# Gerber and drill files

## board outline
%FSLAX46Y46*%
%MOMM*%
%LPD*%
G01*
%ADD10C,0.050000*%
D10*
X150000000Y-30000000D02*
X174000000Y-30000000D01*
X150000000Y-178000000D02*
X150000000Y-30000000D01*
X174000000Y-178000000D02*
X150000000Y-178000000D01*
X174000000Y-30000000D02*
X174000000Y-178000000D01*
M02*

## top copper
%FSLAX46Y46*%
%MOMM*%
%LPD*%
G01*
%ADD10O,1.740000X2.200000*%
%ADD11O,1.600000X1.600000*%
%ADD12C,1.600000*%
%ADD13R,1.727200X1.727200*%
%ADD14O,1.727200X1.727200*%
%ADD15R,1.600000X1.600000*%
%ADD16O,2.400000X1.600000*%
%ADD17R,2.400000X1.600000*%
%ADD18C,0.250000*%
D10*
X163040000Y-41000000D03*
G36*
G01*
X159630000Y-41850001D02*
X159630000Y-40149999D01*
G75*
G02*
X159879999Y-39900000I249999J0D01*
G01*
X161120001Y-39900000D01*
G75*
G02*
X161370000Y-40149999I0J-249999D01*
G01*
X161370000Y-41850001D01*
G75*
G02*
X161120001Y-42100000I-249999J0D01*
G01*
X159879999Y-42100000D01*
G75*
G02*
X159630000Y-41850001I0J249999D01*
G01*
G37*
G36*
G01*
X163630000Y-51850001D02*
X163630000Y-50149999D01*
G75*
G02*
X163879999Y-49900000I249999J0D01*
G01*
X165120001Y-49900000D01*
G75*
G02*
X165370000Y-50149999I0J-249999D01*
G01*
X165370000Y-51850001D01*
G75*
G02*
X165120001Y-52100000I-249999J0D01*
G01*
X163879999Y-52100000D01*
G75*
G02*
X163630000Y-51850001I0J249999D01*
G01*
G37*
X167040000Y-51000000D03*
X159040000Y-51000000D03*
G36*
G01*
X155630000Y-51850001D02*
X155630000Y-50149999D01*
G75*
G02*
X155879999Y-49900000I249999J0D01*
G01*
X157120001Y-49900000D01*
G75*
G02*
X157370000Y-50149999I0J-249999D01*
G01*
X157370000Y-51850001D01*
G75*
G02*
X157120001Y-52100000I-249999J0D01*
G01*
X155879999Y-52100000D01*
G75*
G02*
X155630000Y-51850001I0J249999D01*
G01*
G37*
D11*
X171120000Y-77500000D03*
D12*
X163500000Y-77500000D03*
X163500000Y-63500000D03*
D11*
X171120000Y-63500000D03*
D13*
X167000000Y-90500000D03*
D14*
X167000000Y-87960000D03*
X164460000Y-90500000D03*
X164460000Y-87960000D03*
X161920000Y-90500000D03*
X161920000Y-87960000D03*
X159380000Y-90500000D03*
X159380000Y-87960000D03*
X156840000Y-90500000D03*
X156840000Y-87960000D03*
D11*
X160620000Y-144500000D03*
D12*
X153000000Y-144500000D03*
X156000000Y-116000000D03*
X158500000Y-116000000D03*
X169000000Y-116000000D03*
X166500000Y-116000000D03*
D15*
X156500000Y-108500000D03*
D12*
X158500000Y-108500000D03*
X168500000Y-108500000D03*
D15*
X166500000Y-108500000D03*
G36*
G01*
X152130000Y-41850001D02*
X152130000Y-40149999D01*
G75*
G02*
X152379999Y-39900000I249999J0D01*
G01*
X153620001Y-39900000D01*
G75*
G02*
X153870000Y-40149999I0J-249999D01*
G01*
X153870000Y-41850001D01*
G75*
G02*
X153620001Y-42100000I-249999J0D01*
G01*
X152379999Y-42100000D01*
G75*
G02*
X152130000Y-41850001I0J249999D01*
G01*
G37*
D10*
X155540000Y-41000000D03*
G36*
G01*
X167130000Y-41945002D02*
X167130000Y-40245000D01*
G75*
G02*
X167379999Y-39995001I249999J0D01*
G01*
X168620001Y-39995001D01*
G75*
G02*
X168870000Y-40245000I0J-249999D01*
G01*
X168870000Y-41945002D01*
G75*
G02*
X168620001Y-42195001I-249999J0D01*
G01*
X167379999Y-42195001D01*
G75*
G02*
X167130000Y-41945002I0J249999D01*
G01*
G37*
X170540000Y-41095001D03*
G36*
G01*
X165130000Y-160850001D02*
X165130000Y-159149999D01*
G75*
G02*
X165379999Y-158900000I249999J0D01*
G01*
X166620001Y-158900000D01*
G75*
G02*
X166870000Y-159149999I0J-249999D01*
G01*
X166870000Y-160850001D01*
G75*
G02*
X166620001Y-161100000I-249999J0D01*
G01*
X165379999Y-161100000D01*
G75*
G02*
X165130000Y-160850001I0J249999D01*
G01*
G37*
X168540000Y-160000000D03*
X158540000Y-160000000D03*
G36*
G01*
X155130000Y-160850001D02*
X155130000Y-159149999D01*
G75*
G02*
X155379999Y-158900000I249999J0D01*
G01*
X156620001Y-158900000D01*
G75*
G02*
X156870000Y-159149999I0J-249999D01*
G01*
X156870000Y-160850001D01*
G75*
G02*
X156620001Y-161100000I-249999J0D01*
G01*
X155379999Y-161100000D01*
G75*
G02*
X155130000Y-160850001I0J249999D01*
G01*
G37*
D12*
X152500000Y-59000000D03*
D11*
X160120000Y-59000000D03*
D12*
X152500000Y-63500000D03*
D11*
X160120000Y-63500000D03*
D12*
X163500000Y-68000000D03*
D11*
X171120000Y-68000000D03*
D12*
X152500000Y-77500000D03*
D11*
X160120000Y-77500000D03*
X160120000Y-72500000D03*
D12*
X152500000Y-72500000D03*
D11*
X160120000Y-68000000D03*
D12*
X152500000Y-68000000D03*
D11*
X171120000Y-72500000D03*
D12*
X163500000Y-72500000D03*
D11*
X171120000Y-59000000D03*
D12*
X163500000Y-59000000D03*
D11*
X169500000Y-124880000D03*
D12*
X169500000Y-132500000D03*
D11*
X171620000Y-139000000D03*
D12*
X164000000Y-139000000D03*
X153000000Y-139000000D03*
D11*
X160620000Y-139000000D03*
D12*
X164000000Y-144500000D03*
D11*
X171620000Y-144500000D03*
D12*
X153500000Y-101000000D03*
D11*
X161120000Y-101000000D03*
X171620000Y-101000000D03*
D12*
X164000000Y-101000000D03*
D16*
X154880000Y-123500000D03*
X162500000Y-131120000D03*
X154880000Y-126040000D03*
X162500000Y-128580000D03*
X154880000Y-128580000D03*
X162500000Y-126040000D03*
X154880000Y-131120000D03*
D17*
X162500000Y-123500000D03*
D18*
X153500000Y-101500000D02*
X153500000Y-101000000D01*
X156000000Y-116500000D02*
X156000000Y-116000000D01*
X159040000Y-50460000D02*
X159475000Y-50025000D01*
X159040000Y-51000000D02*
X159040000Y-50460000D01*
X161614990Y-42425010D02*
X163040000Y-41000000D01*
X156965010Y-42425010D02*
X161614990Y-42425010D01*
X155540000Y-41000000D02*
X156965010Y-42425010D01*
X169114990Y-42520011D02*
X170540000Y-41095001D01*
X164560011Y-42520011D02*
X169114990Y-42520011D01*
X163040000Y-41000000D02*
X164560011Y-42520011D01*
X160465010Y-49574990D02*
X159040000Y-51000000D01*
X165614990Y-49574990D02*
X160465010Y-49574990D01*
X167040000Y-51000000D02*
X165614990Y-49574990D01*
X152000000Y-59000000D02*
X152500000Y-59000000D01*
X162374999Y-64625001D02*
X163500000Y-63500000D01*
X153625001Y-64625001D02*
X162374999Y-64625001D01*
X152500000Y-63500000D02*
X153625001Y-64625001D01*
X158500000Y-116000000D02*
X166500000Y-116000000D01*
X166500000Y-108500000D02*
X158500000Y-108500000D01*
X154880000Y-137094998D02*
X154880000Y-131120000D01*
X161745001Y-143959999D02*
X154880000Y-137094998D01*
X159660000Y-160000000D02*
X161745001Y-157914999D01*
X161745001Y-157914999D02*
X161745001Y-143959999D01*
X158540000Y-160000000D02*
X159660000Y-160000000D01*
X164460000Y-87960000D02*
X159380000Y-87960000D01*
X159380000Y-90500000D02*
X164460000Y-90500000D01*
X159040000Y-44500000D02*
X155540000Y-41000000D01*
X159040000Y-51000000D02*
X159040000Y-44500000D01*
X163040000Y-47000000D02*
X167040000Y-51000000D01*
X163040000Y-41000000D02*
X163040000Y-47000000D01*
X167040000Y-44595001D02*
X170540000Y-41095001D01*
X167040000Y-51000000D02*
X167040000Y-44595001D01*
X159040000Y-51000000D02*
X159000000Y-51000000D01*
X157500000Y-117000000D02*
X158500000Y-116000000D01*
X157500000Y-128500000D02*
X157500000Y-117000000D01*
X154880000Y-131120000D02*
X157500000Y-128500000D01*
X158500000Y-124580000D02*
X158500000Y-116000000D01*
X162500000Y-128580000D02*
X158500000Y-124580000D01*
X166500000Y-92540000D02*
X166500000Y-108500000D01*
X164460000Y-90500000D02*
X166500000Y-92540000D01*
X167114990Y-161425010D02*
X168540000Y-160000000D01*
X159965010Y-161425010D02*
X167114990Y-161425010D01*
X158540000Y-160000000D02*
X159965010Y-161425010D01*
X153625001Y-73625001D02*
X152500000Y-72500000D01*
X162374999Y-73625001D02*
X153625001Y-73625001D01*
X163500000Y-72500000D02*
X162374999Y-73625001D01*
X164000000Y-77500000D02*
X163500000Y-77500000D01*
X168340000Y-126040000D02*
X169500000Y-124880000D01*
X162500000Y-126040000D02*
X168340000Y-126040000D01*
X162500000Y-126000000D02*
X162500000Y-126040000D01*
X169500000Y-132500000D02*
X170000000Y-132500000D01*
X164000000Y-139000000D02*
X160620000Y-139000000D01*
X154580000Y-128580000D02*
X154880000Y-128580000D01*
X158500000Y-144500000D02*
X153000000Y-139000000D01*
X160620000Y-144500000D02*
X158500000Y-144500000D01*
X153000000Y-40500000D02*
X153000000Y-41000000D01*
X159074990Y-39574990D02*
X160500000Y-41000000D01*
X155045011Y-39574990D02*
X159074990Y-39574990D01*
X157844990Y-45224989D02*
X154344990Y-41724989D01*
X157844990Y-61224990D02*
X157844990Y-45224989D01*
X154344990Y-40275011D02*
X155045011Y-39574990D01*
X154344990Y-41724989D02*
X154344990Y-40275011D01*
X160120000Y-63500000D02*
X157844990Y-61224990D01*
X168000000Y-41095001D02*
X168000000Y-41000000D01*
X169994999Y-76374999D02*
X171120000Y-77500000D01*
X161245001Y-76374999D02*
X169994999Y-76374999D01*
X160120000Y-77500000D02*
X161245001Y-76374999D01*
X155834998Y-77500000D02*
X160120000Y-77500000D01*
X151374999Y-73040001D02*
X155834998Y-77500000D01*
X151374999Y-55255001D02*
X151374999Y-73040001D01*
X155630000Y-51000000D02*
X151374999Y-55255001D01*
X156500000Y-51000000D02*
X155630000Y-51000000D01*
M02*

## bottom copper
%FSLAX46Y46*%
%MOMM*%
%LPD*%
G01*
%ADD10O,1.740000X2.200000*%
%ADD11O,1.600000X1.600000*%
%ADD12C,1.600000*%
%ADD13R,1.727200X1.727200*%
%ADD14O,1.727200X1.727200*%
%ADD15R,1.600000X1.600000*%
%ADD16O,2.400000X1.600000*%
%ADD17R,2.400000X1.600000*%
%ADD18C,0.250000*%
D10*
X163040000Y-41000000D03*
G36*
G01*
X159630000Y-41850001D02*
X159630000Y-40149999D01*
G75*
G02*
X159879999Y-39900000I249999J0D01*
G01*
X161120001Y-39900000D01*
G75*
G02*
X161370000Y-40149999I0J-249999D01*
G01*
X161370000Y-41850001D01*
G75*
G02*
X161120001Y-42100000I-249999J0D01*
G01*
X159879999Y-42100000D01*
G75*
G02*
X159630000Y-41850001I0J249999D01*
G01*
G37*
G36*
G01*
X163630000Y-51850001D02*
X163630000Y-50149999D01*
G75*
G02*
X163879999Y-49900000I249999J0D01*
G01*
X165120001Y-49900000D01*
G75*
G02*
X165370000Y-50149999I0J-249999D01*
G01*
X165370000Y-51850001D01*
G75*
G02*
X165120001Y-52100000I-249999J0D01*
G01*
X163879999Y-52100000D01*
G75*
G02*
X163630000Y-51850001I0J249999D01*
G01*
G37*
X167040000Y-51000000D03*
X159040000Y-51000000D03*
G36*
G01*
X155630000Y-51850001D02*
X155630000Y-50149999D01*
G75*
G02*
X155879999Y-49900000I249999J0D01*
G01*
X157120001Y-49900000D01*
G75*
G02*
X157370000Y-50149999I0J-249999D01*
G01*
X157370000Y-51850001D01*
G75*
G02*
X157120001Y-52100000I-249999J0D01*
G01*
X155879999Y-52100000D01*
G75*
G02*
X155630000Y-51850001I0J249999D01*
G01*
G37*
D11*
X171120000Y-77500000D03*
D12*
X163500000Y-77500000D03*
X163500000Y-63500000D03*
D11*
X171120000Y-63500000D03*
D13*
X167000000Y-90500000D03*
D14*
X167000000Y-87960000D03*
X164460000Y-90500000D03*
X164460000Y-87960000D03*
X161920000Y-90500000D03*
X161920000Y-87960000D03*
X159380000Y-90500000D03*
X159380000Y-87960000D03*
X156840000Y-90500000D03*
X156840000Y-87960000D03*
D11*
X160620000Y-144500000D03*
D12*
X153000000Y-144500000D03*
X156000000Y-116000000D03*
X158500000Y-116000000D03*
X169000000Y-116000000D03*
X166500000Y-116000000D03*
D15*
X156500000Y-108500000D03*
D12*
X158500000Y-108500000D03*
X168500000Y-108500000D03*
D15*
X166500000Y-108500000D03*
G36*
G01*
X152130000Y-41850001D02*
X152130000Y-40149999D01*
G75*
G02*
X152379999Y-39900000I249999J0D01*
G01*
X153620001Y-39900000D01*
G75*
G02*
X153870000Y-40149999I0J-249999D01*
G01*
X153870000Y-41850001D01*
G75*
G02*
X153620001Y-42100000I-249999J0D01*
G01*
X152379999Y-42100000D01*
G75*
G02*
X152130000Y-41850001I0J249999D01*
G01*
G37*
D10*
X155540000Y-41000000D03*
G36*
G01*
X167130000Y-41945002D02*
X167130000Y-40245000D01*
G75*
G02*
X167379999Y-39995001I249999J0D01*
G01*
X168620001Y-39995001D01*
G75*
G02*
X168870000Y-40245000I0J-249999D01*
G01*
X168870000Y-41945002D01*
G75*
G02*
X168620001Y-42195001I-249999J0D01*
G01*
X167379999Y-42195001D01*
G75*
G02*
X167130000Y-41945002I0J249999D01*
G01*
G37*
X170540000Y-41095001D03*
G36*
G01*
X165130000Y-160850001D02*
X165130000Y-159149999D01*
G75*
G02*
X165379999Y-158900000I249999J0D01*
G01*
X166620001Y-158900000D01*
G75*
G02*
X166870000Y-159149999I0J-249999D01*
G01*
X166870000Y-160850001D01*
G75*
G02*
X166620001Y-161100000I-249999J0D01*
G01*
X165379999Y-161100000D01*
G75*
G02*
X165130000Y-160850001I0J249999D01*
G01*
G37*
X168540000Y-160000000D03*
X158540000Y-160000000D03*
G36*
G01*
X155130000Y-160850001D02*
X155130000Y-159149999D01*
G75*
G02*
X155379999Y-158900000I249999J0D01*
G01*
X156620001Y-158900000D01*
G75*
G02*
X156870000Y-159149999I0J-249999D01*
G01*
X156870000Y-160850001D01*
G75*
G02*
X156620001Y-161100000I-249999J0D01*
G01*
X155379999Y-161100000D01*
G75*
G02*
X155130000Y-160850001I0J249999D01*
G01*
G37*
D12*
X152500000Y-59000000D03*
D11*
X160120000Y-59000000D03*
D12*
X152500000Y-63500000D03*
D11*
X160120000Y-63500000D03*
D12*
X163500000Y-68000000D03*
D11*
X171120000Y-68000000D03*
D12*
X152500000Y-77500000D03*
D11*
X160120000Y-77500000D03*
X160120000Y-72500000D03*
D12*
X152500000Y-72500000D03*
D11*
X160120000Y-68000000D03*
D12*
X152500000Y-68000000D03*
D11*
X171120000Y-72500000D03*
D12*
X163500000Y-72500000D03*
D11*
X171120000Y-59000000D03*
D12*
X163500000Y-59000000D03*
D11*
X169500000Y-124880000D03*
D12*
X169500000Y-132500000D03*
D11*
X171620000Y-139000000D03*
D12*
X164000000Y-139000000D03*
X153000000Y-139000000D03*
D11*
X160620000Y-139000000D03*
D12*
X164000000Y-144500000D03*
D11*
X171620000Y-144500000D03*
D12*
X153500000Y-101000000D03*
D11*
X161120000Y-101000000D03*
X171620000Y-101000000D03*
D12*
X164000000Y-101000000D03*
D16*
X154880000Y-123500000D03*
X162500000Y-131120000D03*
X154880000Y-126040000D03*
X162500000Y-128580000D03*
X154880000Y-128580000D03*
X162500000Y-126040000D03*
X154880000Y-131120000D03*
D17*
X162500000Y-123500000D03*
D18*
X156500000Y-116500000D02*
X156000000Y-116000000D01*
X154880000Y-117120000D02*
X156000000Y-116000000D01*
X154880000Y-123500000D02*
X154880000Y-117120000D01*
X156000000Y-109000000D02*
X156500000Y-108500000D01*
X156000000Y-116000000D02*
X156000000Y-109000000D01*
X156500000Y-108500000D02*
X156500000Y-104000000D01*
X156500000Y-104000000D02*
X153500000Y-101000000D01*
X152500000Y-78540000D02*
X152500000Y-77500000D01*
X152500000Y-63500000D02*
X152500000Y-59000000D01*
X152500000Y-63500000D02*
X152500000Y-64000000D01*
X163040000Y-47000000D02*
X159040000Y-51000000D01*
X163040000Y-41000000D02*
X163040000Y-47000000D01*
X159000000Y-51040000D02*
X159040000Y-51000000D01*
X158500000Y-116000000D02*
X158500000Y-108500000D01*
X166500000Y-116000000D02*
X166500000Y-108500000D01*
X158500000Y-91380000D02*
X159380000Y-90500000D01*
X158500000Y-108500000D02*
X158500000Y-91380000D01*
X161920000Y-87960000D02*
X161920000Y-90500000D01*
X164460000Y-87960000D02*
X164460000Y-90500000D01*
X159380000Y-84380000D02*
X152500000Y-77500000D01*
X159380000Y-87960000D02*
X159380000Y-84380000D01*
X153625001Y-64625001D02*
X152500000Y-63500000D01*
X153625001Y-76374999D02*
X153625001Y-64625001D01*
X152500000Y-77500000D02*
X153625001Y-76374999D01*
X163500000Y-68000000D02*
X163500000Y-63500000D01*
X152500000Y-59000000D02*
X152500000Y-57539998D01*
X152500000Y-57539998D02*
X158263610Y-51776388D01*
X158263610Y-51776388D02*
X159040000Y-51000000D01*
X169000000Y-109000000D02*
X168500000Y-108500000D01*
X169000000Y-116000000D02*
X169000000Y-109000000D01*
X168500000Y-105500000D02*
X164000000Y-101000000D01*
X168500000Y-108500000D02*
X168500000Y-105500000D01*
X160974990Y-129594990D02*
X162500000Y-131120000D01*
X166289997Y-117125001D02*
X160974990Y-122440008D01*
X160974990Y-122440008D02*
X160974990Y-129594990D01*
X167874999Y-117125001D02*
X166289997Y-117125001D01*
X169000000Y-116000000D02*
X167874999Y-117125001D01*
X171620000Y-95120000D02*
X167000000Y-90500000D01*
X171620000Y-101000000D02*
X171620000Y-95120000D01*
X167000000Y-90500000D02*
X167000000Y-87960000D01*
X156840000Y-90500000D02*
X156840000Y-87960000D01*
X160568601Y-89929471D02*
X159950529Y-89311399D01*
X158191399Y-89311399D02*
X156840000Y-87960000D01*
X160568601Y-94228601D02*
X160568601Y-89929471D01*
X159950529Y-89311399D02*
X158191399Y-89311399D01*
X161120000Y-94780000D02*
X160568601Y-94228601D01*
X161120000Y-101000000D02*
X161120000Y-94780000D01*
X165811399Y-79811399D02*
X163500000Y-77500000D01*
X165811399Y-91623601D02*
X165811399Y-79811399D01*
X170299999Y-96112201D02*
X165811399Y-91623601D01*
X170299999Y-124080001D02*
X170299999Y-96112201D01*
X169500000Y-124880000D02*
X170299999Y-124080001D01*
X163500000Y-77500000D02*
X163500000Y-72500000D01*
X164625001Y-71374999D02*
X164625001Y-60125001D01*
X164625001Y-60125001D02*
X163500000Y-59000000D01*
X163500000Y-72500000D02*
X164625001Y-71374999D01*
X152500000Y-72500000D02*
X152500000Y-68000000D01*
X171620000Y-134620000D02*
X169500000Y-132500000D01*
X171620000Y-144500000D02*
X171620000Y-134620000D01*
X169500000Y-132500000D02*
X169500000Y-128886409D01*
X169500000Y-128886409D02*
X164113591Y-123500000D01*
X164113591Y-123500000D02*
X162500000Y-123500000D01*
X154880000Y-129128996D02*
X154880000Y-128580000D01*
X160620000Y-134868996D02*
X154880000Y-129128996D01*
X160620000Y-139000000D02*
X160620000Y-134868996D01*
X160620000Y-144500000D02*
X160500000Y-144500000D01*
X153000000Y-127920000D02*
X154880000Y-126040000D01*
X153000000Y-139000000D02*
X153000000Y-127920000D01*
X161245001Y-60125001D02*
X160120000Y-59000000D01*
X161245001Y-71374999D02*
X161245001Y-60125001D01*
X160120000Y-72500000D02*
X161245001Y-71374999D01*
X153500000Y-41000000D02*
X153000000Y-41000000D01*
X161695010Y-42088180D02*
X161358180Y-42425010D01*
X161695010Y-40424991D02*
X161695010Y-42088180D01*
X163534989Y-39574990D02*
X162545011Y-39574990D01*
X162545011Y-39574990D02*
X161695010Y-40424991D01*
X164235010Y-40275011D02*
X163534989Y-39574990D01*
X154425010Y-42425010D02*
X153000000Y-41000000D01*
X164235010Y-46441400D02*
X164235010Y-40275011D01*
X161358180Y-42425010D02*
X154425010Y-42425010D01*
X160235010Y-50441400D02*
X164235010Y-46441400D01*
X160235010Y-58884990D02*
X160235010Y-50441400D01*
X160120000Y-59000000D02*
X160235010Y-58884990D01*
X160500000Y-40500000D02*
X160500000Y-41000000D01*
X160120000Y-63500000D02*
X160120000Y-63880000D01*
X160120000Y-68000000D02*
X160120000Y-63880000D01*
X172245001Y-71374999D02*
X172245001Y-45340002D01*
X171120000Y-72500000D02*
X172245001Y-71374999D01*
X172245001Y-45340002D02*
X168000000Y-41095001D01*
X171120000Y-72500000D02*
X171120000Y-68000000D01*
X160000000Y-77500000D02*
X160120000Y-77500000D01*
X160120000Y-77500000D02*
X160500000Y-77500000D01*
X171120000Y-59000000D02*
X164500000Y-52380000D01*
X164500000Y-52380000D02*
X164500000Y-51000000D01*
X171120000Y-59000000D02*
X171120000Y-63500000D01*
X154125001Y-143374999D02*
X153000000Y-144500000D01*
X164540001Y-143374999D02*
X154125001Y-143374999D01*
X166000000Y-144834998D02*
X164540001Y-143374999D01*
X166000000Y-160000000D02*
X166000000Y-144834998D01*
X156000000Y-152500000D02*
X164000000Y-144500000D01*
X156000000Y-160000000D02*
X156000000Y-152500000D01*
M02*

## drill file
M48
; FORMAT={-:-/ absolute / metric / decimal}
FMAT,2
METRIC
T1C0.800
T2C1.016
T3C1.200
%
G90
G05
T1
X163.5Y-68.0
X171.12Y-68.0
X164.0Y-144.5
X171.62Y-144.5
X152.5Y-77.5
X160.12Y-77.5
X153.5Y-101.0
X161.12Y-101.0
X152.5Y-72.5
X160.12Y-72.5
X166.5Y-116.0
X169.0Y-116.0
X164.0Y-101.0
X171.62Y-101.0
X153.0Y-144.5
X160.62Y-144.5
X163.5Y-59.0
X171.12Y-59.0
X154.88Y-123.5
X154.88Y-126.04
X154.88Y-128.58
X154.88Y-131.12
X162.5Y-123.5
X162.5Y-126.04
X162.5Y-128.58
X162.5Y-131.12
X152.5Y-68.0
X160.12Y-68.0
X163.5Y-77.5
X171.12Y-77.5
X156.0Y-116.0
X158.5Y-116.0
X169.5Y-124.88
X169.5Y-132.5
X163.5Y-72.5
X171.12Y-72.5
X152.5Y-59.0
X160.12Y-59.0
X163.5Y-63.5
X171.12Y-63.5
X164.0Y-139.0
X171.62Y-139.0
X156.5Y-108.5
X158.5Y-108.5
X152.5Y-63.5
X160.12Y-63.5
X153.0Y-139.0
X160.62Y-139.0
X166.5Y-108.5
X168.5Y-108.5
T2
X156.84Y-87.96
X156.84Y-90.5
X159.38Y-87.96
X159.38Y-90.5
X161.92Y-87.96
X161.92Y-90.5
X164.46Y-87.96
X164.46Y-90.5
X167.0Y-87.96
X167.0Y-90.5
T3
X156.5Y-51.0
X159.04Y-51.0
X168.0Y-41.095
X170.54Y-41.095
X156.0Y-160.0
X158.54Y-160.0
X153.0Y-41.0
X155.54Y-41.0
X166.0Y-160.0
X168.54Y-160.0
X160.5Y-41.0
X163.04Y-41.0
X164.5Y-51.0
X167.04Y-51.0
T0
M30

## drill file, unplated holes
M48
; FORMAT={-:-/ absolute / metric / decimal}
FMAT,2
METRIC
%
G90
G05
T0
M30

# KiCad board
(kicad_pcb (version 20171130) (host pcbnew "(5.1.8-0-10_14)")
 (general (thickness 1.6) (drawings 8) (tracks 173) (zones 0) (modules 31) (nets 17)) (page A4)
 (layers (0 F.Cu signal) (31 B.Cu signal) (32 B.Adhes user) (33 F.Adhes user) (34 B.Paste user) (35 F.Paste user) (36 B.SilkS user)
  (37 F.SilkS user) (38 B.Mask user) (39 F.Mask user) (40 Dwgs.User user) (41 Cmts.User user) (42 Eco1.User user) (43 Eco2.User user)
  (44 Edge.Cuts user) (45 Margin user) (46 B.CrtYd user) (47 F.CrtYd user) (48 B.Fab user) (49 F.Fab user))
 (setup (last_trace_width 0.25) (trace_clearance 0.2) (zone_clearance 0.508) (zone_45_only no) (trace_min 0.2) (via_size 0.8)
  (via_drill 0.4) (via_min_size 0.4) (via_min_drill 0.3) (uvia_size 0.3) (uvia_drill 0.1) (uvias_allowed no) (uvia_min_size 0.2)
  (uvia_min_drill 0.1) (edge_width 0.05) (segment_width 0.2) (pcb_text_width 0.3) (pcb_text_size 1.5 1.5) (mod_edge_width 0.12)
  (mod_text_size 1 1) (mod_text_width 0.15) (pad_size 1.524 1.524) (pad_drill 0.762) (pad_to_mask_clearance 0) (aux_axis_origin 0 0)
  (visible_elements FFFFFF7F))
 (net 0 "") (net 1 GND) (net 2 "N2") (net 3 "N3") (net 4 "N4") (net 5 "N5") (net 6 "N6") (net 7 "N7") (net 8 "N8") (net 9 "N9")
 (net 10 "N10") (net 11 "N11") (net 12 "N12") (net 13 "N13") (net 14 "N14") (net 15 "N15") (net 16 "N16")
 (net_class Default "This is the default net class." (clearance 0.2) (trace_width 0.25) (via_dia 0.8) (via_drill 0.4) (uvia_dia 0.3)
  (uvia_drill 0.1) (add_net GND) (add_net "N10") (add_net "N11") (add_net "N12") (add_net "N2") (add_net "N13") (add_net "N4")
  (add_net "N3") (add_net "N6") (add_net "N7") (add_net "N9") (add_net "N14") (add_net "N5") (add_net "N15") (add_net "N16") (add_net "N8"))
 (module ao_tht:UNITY (layer F.Cu) (at 162 105 270)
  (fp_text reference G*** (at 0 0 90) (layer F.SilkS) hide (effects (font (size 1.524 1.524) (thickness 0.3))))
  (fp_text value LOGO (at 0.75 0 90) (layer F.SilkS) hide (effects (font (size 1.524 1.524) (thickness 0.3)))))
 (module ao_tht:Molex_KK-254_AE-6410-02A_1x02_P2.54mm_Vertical (layer F.Cu) (at 160.5 41)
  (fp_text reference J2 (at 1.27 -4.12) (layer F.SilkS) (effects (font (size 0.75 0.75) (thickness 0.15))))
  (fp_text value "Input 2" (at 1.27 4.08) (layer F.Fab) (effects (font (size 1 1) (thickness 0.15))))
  (pad 2 thru_hole oval (at 2.54 0) (size 1.74 2.2) (drill 1.2) (layers *.Cu *.Mask) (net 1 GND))
  (pad 1 thru_hole roundrect (at 0 0) (size 1.74 2.2) (drill 1.2) (layers *.Cu *.Mask) (roundrect_rratio 0.1436775862068966) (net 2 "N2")))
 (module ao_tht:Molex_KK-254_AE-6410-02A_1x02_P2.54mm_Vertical (layer F.Cu) (at 164.5 51)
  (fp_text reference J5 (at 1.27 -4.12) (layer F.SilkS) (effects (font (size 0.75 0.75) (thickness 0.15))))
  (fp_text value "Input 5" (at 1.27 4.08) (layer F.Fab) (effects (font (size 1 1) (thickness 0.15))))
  (pad 1 thru_hole roundrect (at 0 0) (size 1.74 2.2) (drill 1.2) (layers *.Cu *.Mask) (roundrect_rratio 0.1436775862068966) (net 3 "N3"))
  (pad 2 thru_hole oval (at 2.54 0) (size 1.74 2.2) (drill 1.2) (layers *.Cu *.Mask) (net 1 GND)))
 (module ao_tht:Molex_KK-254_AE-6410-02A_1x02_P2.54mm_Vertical (layer F.Cu) (at 156.5 51)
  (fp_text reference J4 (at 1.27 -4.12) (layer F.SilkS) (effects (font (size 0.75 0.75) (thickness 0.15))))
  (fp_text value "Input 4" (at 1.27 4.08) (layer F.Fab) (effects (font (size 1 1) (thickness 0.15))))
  (pad 2 thru_hole oval (at 2.54 0) (size 1.74 2.2) (drill 1.2) (layers *.Cu *.Mask) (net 1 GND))
  (pad 1 thru_hole roundrect (at 0 0) (size 1.74 2.2) (drill 1.2) (layers *.Cu *.Mask) (roundrect_rratio 0.1436775862068966) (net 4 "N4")))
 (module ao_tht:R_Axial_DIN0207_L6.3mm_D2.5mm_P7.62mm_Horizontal (layer B.Cu) (at 163.5 77.5)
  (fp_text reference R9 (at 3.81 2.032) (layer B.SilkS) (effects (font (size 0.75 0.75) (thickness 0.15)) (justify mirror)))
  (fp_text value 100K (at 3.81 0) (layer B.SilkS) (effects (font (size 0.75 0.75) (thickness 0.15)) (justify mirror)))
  (pad 2 thru_hole oval (at 7.62 0) (size 1.6 1.6) (drill 0.8) (layers *.Cu *.Mask) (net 4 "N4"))
  (pad 1 thru_hole circle (at 0 0) (size 1.6 1.6) (drill 0.8) (layers *.Cu *.Mask) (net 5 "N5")))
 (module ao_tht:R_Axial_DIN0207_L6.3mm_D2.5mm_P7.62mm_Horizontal (layer B.Cu) (at 163.5 63.5)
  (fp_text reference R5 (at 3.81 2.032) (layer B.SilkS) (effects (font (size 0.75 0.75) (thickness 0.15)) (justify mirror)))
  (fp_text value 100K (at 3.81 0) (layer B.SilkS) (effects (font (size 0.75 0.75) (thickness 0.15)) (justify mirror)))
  (pad 1 thru_hole circle (at 0 0) (size 1.6 1.6) (drill 0.8) (layers *.Cu *.Mask) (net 1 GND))
  (pad 2 thru_hole oval (at 7.62 0) (size 1.6 1.6) (drill 0.8) (layers *.Cu *.Mask) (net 3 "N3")))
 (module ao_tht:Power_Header (layer B.Cu) (at 167 90.5 90)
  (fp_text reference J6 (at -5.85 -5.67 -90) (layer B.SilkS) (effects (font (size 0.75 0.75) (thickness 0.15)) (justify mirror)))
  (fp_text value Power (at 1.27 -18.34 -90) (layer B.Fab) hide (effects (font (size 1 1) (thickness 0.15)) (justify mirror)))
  (pad 1 thru_hole rect (at 0 0 90) (size 1.7272 1.7272) (drill 1.016) (layers *.Cu *.Mask) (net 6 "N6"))
  (pad 2 thru_hole oval (at 2.54 0 90) (size 1.7272 1.7272) (drill 1.016) (layers *.Cu *.Mask) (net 6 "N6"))
  (pad 3 thru_hole oval (at 0 -2.54 90) (size 1.7272 1.7272) (drill 1.016) (layers *.Cu *.Mask) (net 1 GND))
  (pad 4 thru_hole oval (at 2.54 -2.54 90) (size 1.7272 1.7272) (drill 1.016) (layers *.Cu *.Mask) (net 1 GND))
  (pad 5 thru_hole oval (at 0 -5.08 90) (size 1.7272 1.7272) (drill 1.016) (layers *.Cu *.Mask) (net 1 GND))
  (pad 6 thru_hole oval (at 2.54 -5.08 90) (size 1.7272 1.7272) (drill 1.016) (layers *.Cu *.Mask) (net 1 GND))
  (pad 7 thru_hole oval (at 0 -7.62 90) (size 1.7272 1.7272) (drill 1.016) (layers *.Cu *.Mask) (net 1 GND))
  (pad 8 thru_hole oval (at 2.54 -7.62 90) (size 1.7272 1.7272) (drill 1.016) (layers *.Cu *.Mask) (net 1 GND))
  (pad 9 thru_hole oval (at 0 -10.16 90) (size 1.7272 1.7272) (drill 1.016) (layers *.Cu *.Mask) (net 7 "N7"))
  (pad 10 thru_hole oval (at 2.54 -10.16 90) (size 1.7272 1.7272) (drill 1.016) (layers *.Cu *.Mask) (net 7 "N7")))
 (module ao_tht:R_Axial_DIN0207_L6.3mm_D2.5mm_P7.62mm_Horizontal (layer B.Cu) (at 153 144.5)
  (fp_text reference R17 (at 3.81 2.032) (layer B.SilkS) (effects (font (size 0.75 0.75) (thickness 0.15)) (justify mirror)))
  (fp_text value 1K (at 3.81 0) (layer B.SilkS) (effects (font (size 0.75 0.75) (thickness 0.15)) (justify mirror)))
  (pad 2 thru_hole oval (at 7.62 0) (size 1.6 1.6) (drill 0.8) (layers *.Cu *.Mask) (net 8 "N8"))
  (pad 1 thru_hole circle (at 0 0) (size 1.6 1.6) (drill 0.8) (layers *.Cu *.Mask) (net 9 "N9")))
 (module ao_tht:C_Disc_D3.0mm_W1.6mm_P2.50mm (layer B.Cu) (at 156 116)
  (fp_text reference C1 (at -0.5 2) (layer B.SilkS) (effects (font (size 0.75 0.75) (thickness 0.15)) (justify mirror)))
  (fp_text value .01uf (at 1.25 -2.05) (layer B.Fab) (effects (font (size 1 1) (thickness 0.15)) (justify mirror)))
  (pad 1 thru_hole circle (at 0 0) (size 1.6 1.6) (drill 0.8) (layers *.Cu *.Mask) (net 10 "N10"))
  (pad 2 thru_hole circle (at 2.5 0) (size 1.6 1.6) (drill 0.8) (layers *.Cu *.Mask) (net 1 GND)))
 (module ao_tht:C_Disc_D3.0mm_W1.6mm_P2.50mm (layer B.Cu) (at 166.5 116)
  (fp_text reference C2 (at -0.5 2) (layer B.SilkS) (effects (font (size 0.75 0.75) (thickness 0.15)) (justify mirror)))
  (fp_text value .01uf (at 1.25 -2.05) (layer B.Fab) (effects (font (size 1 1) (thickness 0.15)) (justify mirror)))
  (pad 2 thru_hole circle (at 2.5 0) (size 1.6 1.6) (drill 0.8) (layers *.Cu *.Mask) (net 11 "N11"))
  (pad 1 thru_hole circle (at 0 0) (size 1.6 1.6) (drill 0.8) (layers *.Cu *.Mask) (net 1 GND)))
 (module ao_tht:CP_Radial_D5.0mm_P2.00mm (layer B.Cu) (at 156.5 108.5)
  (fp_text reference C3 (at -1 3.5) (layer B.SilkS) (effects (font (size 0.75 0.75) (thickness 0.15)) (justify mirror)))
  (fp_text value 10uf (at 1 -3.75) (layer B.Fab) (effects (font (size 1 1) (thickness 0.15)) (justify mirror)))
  (pad 1 thru_hole rect (at 0 0) (size 1.6 1.6) (drill 0.8) (layers *.Cu *.Mask) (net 10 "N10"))
  (pad 2 thru_hole circle (at 2 0) (size 1.6 1.6) (drill 0.8) (layers *.Cu *.Mask) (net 1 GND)))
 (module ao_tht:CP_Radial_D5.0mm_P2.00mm (layer B.Cu) (at 166.5 108.5)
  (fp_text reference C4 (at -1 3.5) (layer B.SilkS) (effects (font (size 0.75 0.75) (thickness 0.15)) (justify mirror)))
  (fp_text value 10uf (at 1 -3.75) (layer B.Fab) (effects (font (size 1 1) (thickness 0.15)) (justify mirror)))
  (pad 2 thru_hole circle (at 2 0) (size 1.6 1.6) (drill 0.8) (layers *.Cu *.Mask) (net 11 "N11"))
  (pad 1 thru_hole rect (at 0 0) (size 1.6 1.6) (drill 0.8) (layers *.Cu *.Mask) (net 1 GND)))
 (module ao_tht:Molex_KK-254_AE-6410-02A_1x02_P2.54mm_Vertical (layer F.Cu) (at 153 41)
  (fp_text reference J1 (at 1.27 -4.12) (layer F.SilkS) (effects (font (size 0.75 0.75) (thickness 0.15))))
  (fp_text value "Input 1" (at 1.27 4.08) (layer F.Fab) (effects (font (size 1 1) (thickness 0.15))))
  (pad 1 thru_hole roundrect (at 0 0) (size 1.74 2.2) (drill 1.2) (layers *.Cu *.Mask) (roundrect_rratio 0.1436775862068966) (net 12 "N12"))
  (pad 2 thru_hole oval (at 2.54 0) (size 1.74 2.2) (drill 1.2) (layers *.Cu *.Mask) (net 1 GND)))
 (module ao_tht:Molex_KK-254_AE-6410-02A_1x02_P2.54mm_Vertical (layer F.Cu) (at 168 41.095001)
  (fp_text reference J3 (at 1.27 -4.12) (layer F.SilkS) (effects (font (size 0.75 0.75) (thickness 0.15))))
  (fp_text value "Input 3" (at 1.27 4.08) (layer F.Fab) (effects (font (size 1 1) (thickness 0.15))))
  (pad 1 thru_hole roundrect (at 0 0) (size 1.74 2.2) (drill 1.2) (layers *.Cu *.Mask) (roundrect_rratio 0.1436775862068966) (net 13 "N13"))
  (pad 2 thru_hole oval (at 2.54 0) (size 1.74 2.2) (drill 1.2) (layers *.Cu *.Mask) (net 1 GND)))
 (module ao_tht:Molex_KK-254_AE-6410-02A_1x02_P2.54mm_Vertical (layer F.Cu) (at 166 160)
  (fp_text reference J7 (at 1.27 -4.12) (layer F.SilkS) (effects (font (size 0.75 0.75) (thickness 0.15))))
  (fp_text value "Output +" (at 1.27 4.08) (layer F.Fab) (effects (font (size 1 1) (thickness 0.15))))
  (pad 1 thru_hole roundrect (at 0 0) (size 1.74 2.2) (drill 1.2) (layers *.Cu *.Mask) (roundrect_rratio 0.1436775862068966) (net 9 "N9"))
  (pad 2 thru_hole oval (at 2.54 0) (size 1.74 2.2) (drill 1.2) (layers *.Cu *.Mask) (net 1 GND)))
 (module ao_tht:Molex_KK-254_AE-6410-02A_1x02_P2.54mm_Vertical (layer F.Cu) (at 156 160)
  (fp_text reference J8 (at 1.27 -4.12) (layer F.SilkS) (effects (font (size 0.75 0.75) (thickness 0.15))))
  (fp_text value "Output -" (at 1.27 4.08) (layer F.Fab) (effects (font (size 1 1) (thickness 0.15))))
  (pad 2 thru_hole oval (at 2.54 0) (size 1.74 2.2) (drill 1.2) (layers *.Cu *.Mask) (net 1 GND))
  (pad 1 thru_hole roundrect (at 0 0) (size 1.74 2.2) (drill 1.2) (layers *.Cu *.Mask) (roundrect_rratio 0.1436775862068966) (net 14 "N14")))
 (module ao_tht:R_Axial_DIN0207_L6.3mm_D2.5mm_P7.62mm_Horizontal (layer B.Cu) (at 152.5 59)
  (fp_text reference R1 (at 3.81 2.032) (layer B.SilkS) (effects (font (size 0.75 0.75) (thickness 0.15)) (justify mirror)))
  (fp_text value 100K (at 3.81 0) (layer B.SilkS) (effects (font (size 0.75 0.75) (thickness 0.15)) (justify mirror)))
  (pad 1 thru_hole circle (at 0 0) (size 1.6 1.6) (drill 0.8) (layers *.Cu *.Mask) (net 1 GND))
  (pad 2 thru_hole oval (at 7.62 0) (size 1.6 1.6) (drill 0.8) (layers *.Cu *.Mask) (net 12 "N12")))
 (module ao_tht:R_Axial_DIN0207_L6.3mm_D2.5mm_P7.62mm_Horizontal (layer B.Cu) (at 152.5 63.5)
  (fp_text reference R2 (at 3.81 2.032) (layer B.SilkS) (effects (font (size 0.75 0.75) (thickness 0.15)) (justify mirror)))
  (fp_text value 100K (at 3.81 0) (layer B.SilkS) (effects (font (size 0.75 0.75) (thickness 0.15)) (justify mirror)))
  (pad 1 thru_hole circle (at 0 0) (size 1.6 1.6) (drill 0.8) (layers *.Cu *.Mask) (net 1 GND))
  (pad 2 thru_hole oval (at 7.62 0) (size 1.6 1.6) (drill 0.8) (layers *.Cu *.Mask) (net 2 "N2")))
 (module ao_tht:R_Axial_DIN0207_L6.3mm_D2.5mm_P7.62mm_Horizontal (layer B.Cu) (at 163.5 68)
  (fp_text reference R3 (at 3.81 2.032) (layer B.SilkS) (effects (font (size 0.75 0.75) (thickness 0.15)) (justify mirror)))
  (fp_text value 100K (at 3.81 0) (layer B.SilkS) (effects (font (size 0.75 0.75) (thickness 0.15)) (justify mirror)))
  (pad 1 thru_hole circle (at 0 0) (size 1.6 1.6) (drill 0.8) (layers *.Cu *.Mask) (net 1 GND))
  (pad 2 thru_hole oval (at 7.62 0) (size 1.6 1.6) (drill 0.8) (layers *.Cu *.Mask) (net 13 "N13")))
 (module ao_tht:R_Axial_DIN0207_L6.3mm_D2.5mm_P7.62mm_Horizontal (layer B.Cu) (at 152.5 77.5)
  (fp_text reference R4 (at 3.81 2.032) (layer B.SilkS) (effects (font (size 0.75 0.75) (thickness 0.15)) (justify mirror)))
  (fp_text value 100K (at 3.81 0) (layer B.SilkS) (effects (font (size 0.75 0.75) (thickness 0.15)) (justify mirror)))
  (pad 1 thru_hole circle (at 0 0) (size 1.6 1.6) (drill 0.8) (layers *.Cu *.Mask) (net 1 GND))
  (pad 2 thru_hole oval (at 7.62 0) (size 1.6 1.6) (drill 0.8) (layers *.Cu *.Mask) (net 4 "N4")))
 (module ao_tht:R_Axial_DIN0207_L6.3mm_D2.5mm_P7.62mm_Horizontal (layer B.Cu) (at 152.5 72.5)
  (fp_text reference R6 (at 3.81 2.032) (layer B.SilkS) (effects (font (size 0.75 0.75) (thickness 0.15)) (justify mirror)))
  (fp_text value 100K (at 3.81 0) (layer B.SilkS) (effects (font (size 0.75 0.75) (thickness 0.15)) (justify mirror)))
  (pad 2 thru_hole oval (at 7.62 0) (size 1.6 1.6) (drill 0.8) (layers *.Cu *.Mask) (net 12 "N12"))
  (pad 1 thru_hole circle (at 0 0) (size 1.6 1.6) (drill 0.8) (layers *.Cu *.Mask) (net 5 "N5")))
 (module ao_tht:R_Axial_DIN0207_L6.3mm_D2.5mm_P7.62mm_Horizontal (layer B.Cu) (at 152.5 68)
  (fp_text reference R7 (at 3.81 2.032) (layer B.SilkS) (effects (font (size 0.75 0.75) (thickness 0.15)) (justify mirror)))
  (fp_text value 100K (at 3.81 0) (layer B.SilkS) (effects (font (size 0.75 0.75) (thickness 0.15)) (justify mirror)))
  (pad 2 thru_hole oval (at 7.62 0) (size 1.6 1.6) (drill 0.8) (layers *.Cu *.Mask) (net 2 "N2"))
  (pad 1 thru_hole circle (at 0 0) (size 1.6 1.6) (drill 0.8) (layers *.Cu *.Mask) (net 5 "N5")))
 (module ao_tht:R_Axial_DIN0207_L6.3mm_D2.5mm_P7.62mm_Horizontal (layer B.Cu) (at 163.5 72.5)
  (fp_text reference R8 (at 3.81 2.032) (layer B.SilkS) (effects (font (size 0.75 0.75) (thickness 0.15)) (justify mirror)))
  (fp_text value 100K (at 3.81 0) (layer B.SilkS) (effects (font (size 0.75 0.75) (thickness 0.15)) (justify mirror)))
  (pad 2 thru_hole oval (at 7.62 0) (size 1.6 1.6) (drill 0.8) (layers *.Cu *.Mask) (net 13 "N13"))
  (pad 1 thru_hole circle (at 0 0) (size 1.6 1.6) (drill 0.8) (layers *.Cu *.Mask) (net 5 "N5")))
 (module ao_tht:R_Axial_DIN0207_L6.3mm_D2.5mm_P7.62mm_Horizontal (layer B.Cu) (at 163.5 59)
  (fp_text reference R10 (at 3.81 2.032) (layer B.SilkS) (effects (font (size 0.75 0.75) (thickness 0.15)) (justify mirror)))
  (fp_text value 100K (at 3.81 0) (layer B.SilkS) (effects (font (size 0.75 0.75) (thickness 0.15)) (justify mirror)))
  (pad 2 thru_hole oval (at 7.62 0) (size 1.6 1.6) (drill 0.8) (layers *.Cu *.Mask) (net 3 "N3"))
  (pad 1 thru_hole circle (at 0 0) (size 1.6 1.6) (drill 0.8) (layers *.Cu *.Mask) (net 5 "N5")))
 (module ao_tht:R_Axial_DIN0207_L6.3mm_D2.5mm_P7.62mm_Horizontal (layer B.Cu) (at 169.5 132.5 90)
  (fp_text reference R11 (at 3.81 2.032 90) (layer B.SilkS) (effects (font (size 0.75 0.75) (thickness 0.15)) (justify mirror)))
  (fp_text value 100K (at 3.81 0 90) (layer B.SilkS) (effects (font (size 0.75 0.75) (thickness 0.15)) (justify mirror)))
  (pad 2 thru_hole oval (at 7.62 0 90) (size 1.6 1.6) (drill 0.8) (layers *.Cu *.Mask) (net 5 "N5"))
  (pad 1 thru_hole circle (at 0 0 90) (size 1.6 1.6) (drill 0.8) (layers *.Cu *.Mask) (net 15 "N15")))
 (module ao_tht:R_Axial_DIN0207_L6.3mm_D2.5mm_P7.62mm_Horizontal (layer B.Cu) (at 164 139)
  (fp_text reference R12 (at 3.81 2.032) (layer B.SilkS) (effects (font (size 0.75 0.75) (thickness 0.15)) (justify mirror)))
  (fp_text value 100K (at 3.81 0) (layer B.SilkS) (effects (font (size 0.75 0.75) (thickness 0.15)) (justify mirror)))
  (pad 2 thru_hole oval (at 7.62 0) (size 1.6 1.6) (drill 0.8) (layers *.Cu *.Mask) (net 15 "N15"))
  (pad 1 thru_hole circle (at 0 0) (size 1.6 1.6) (drill 0.8) (layers *.Cu *.Mask) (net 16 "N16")))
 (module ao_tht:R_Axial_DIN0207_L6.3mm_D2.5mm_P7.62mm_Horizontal (layer B.Cu) (at 153 139)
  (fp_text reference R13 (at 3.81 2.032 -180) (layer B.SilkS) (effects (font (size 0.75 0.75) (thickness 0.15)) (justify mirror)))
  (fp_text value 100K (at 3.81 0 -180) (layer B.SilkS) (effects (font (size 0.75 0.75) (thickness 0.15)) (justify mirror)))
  (pad 1 thru_hole circle (at 0 0) (size 1.6 1.6) (drill 0.8) (layers *.Cu *.Mask) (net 8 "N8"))
  (pad 2 thru_hole oval (at 7.62 0) (size 1.6 1.6) (drill 0.8) (layers *.Cu *.Mask) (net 16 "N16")))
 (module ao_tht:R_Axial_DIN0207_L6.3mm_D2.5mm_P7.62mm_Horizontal (layer B.Cu) (at 164 144.5)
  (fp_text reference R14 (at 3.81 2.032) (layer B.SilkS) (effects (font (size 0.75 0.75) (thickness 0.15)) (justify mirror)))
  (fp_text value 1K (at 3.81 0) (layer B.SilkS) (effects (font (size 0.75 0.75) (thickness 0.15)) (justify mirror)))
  (pad 1 thru_hole circle (at 0 0) (size 1.6 1.6) (drill 0.8) (layers *.Cu *.Mask) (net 14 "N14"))
  (pad 2 thru_hole oval (at 7.62 0) (size 1.6 1.6) (drill 0.8) (layers *.Cu *.Mask) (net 15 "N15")))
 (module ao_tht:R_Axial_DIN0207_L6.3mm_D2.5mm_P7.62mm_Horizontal (layer B.Cu) (at 153.5 101)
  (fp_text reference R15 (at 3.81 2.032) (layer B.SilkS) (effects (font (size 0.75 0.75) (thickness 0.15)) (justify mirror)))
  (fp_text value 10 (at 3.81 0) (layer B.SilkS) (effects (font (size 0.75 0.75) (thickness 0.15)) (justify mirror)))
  (pad 1 thru_hole circle (at 0 0) (size 1.6 1.6) (drill 0.8) (layers *.Cu *.Mask) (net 10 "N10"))
  (pad 2 thru_hole oval (at 7.62 0) (size 1.6 1.6) (drill 0.8) (layers *.Cu *.Mask) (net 7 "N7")))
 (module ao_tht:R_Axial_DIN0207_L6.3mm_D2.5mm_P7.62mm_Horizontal (layer B.Cu) (at 164 101)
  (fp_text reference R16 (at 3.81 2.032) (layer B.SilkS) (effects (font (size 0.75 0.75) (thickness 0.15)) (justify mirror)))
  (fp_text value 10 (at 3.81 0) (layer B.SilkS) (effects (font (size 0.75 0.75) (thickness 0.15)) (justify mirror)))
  (pad 2 thru_hole oval (at 7.62 0) (size 1.6 1.6) (drill 0.8) (layers *.Cu *.Mask) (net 6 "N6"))
  (pad 1 thru_hole circle (at 0 0) (size 1.6 1.6) (drill 0.8) (layers *.Cu *.Mask) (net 11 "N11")))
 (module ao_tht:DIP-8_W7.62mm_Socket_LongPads (layer B.Cu) (at 162.5 123.5 180)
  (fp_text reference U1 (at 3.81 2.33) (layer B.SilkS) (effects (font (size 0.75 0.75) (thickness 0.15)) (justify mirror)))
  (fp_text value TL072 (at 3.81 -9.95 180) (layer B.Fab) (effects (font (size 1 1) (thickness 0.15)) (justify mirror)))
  (pad 8 thru_hole oval (at 7.62 0 180) (size 2.4 1.6) (drill 0.8) (layers *.Cu *.Mask) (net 10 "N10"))
  (pad 4 thru_hole oval (at 0 -7.62 180) (size 2.4 1.6) (drill 0.8) (layers *.Cu *.Mask) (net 11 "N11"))
  (pad 7 thru_hole oval (at 7.62 -2.54 180) (size 2.4 1.6) (drill 0.8) (layers *.Cu *.Mask) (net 8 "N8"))
  (pad 3 thru_hole oval (at 0 -5.08 180) (size 2.4 1.6) (drill 0.8) (layers *.Cu *.Mask) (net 1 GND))
  (pad 6 thru_hole oval (at 7.62 -5.08 180) (size 2.4 1.6) (drill 0.8) (layers *.Cu *.Mask) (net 16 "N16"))
  (pad 2 thru_hole oval (at 0 -2.54 180) (size 2.4 1.6) (drill 0.8) (layers *.Cu *.Mask) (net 5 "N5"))
  (pad 5 thru_hole oval (at 7.62 -7.62 180) (size 2.4 1.6) (drill 0.8) (layers *.Cu *.Mask) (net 1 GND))
  (pad 1 thru_hole rect (at 0 0 180) (size 2.4 1.6) (drill 0.8) (layers *.Cu *.Mask) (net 15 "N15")))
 (gr_line (start 150 30) (end 174 30) (layer Edge.Cuts) (width 0.05))
 (gr_line (start 150 178) (end 150 30) (layer Edge.Cuts) (width 0.05))
 (gr_line (start 174 178) (end 150 178) (layer Edge.Cuts) (width 0.05))
 (gr_line (start 174 30) (end 174 178) (layer Edge.Cuts) (width 0.05))
 (segment (start 156.5 116.5) (end 156 116) (width 0.25) (layer B.Cu) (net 10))
 (segment (start 153.5 101.5) (end 153.5 101) (width 0.25) (layer F.Cu) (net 10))
 (segment (start 156 116.5) (end 156 116) (width 0.25) (layer F.Cu) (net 10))
 (segment (start 154.88 117.12) (end 156 116) (width 0.25) (layer B.Cu) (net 10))
 (segment (start 154.88 123.5) (end 154.88 117.12) (width 0.25) (layer B.Cu) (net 10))
 (segment (start 156 109) (end 156.5 108.5) (width 0.25) (layer B.Cu) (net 10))
 (segment (start 156 116) (end 156 109) (width 0.25) (layer B.Cu) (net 10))
 (segment (start 156.5 108.5) (end 156.5 104) (width 0.25) (layer B.Cu) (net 10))
 (segment (start 156.5 104) (end 153.5 101) (width 0.25) (layer B.Cu) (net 10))
 (segment (start 159.04 50.46) (end 159.475 50.025) (width 0.25) (layer F.Cu) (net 1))
 (segment (start 159.04 51) (end 159.04 50.46) (width 0.25) (layer F.Cu) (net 1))
 (segment (start 152.5 78.54) (end 152.5 77.5) (width 0.25) (layer B.Cu) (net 1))
 (segment (start 152.5 63.5) (end 152.5 59) (width 0.25) (layer B.Cu) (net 1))
 (segment (start 152.5 63.5) (end 152.5 64) (width 0.25) (layer B.Cu) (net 1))
 (segment (start 163.04 47) (end 159.04 51) (width 0.25) (layer B.Cu) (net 1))
 (segment (start 163.04 41) (end 163.04 47) (width 0.25) (layer B.Cu) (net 1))
 (segment (start 159 51.04) (end 159.04 51) (width 0.25) (layer B.Cu) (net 1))
 (segment (start 161.61499 42.42501) (end 163.04 41) (width 0.25) (layer F.Cu) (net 1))
 (segment (start 156.96501 42.42501) (end 161.61499 42.42501) (width 0.25) (layer F.Cu) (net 1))
 (segment (start 155.54 41) (end 156.96501 42.42501) (width 0.25) (layer F.Cu) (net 1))
 (segment (start 169.11499 42.520011) (end 170.54 41.095001) (width 0.25) (layer F.Cu) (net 1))
 (segment (start 164.560011 42.520011) (end 169.11499 42.520011) (width 0.25) (layer F.Cu) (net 1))
 (segment (start 163.04 41) (end 164.560011 42.520011) (width 0.25) (layer F.Cu) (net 1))
 (segment (start 160.46501 49.57499) (end 159.04 51) (width 0.25) (layer F.Cu) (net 1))
 (segment (start 165.61499 49.57499) (end 160.46501 49.57499) (width 0.25) (layer F.Cu) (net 1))
 (segment (start 167.04 51) (end 165.61499 49.57499) (width 0.25) (layer F.Cu) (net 1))
 (segment (start 152 59) (end 152.5 59) (width 0.25) (layer F.Cu) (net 1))
 (segment (start 162.374999 64.625001) (end 163.5 63.5) (width 0.25) (layer F.Cu) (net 1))
 (segment (start 153.625001 64.625001) (end 162.374999 64.625001) (width 0.25) (layer F.Cu) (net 1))
 (segment (start 152.5 63.5) (end 153.625001 64.625001) (width 0.25) (layer F.Cu) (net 1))
 (segment (start 158.5 116) (end 166.5 116) (width 0.25) (layer F.Cu) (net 1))
 (segment (start 166.5 108.5) (end 158.5 108.5) (width 0.25) (layer F.Cu) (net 1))
 (segment (start 154.88 137.094998) (end 154.88 131.12) (width 0.25) (layer F.Cu) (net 1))
 (segment (start 161.745001 143.959999) (end 154.88 137.094998) (width 0.25) (layer F.Cu) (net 1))
 (segment (start 159.66 160) (end 161.745001 157.914999) (width 0.25) (layer F.Cu) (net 1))
 (segment (start 161.745001 157.914999) (end 161.745001 143.959999) (width 0.25) (layer F.Cu) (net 1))
 (segment (start 158.54 160) (end 159.66 160) (width 0.25) (layer F.Cu) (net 1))
 (segment (start 158.5 116) (end 158.5 108.5) (width 0.25) (layer B.Cu) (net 1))
 (segment (start 166.5 116) (end 166.5 108.5) (width 0.25) (layer B.Cu) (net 1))
 (segment (start 158.5 91.38) (end 159.38 90.5) (width 0.25) (layer B.Cu) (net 1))
 (segment (start 158.5 108.5) (end 158.5 91.38) (width 0.25) (layer B.Cu) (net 1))
 (segment (start 164.46 87.96) (end 159.38 87.96) (width 0.25) (layer F.Cu) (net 1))
 (segment (start 159.38 90.5) (end 164.46 90.5) (width 0.25) (layer F.Cu) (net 1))
 (segment (start 161.92 87.96) (end 161.92 90.5) (width 0.25) (layer B.Cu) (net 1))
 (segment (start 164.46 87.96) (end 164.46 90.5) (width 0.25) (layer B.Cu) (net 1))
 (segment (start 159.38 84.38) (end 152.5 77.5) (width 0.25) (layer B.Cu) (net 1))
 (segment (start 159.38 87.96) (end 159.38 84.38) (width 0.25) (layer B.Cu) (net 1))
 (segment (start 153.625001 64.625001) (end 152.5 63.5) (width 0.25) (layer B.Cu) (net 1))
 (segment (start 153.625001 76.374999) (end 153.625001 64.625001) (width 0.25) (layer B.Cu) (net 1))
 (segment (start 152.5 77.5) (end 153.625001 76.374999) (width 0.25) (layer B.Cu) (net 1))
 (segment (start 163.5 68) (end 163.5 63.5) (width 0.25) (layer B.Cu) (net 1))
 (segment (start 152.5 59) (end 152.5 57.539998) (width 0.25) (layer B.Cu) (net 1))
 (segment (start 152.5 57.539998) (end 158.26361 51.776388) (width 0.25) (layer B.Cu) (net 1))
 (segment (start 158.26361 51.776388) (end 159.04 51) (width 0.25) (layer B.Cu) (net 1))
 (segment (start 159.04 44.5) (end 155.54 41) (width 0.25) (layer F.Cu) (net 1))
 (segment (start 159.04 51) (end 159.04 44.5) (width 0.25) (layer F.Cu) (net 1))
 (segment (start 163.04 47) (end 167.04 51) (width 0.25) (layer F.Cu) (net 1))
 (segment (start 163.04 41) (end 163.04 47) (width 0.25) (layer F.Cu) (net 1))
 (segment (start 167.04 44.595001) (end 170.54 41.095001) (width 0.25) (layer F.Cu) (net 1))
 (segment (start 167.04 51) (end 167.04 44.595001) (width 0.25) (layer F.Cu) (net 1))
 (segment (start 159.04 51) (end 159 51) (width 0.25) (layer F.Cu) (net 1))
 (segment (start 157.5 117) (end 158.5 116) (width 0.25) (layer F.Cu) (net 1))
 (segment (start 157.5 128.5) (end 157.5 117) (width 0.25) (layer F.Cu) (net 1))
 (segment (start 154.88 131.12) (end 157.5 128.5) (width 0.25) (layer F.Cu) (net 1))
 (segment (start 158.5 124.58) (end 158.5 116) (width 0.25) (layer F.Cu) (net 1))
 (segment (start 162.5 128.58) (end 158.5 124.58) (width 0.25) (layer F.Cu) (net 1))
 (segment (start 166.5 92.54) (end 166.5 108.5) (width 0.25) (layer F.Cu) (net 1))
 (segment (start 164.46 90.5) (end 166.5 92.54) (width 0.25) (layer F.Cu) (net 1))
 (segment (start 167.11499 161.42501) (end 168.54 160) (width 0.25) (layer F.Cu) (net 1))
 (segment (start 159.96501 161.42501) (end 167.11499 161.42501) (width 0.25) (layer F.Cu) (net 1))
 (segment (start 158.54 160) (end 159.96501 161.42501) (width 0.25) (layer F.Cu) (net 1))
 (segment (start 169 109) (end 168.5 108.5) (width 0.25) (layer B.Cu) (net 11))
 (segment (start 169 116) (end 169 109) (width 0.25) (layer B.Cu) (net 11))
 (segment (start 168.5 105.5) (end 164 101) (width 0.25) (layer B.Cu) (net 11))
 (segment (start 168.5 108.5) (end 168.5 105.5) (width 0.25) (layer B.Cu) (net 11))
 (segment (start 160.97499 129.59499) (end 162.5 131.12) (width 0.25) (layer B.Cu) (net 11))
 (segment (start 166.289997 117.125001) (end 160.97499 122.440008) (width 0.25) (layer B.Cu) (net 11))
 (segment (start 160.97499 122.440008) (end 160.97499 129.59499) (width 0.25) (layer B.Cu) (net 11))
 (segment (start 167.874999 117.125001) (end 166.289997 117.125001) (width 0.25) (layer B.Cu) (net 11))
 (segment (start 169 116) (end 167.874999 117.125001) (width 0.25) (layer B.Cu) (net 11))
 (segment (start 171.62 95.12) (end 167 90.5) (width 0.25) (layer B.Cu) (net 6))
 (segment (start 171.62 101) (end 171.62 95.12) (width 0.25) (layer B.Cu) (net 6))
 (segment (start 167 90.5) (end 167 87.96) (width 0.25) (layer B.Cu) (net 6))
 (segment (start 156.84 90.5) (end 156.84 87.96) (width 0.25) (layer B.Cu) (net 7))
 (segment (start 160.568601 89.929471) (end 159.950529 89.311399) (width 0.25) (layer B.Cu) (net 7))
 (segment (start 158.191399 89.311399) (end 156.84 87.96) (width 0.25) (layer B.Cu) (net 7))
 (segment (start 160.568601 94.228601) (end 160.568601 89.929471) (width 0.25) (layer B.Cu) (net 7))
 (segment (start 159.950529 89.311399) (end 158.191399 89.311399) (width 0.25) (layer B.Cu) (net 7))
 (segment (start 161.12 94.78) (end 160.568601 94.228601) (width 0.25) (layer B.Cu) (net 7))
 (segment (start 161.12 101) (end 161.12 94.78) (width 0.25) (layer B.Cu) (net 7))
 (segment (start 153.625001 73.625001) (end 152.5 72.5) (width 0.25) (layer F.Cu) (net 5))
 (segment (start 162.374999 73.625001) (end 153.625001 73.625001) (width 0.25) (layer F.Cu) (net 5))
 (segment (start 163.5 72.5) (end 162.374999 73.625001) (width 0.25) (layer F.Cu) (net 5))
 (segment (start 164 77.5) (end 163.5 77.5) (width 0.25) (layer F.Cu) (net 5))
 (segment (start 168.34 126.04) (end 169.5 124.88) (width 0.25) (layer F.Cu) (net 5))
 (segment (start 162.5 126.04) (end 168.34 126.04) (width 0.25) (layer F.Cu) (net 5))
 (segment (start 165.811399 79.811399) (end 163.5 77.5) (width 0.25) (layer B.Cu) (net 5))
 (segment (start 165.811399 91.623601) (end 165.811399 79.811399) (width 0.25) (layer B.Cu) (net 5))
 (segment (start 170.299999 96.112201) (end 165.811399 91.623601) (width 0.25) (layer B.Cu) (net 5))
 (segment (start 170.299999 124.080001) (end 170.299999 96.112201) (width 0.25) (layer B.Cu) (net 5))
 (segment (start 169.5 124.88) (end 170.299999 124.080001) (width 0.25) (layer B.Cu) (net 5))
 (segment (start 162.5 126) (end 162.5 126.04) (width 0.25) (layer F.Cu) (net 5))
 (segment (start 163.5 77.5) (end 163.5 72.5) (width 0.25) (layer B.Cu) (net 5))
 (segment (start 164.625001 71.374999) (end 164.625001 60.125001) (width 0.25) (layer B.Cu) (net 5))
 (segment (start 164.625001 60.125001) (end 163.5 59) (width 0.25) (layer B.Cu) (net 5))
 (segment (start 163.5 72.5) (end 164.625001 71.374999) (width 0.25) (layer B.Cu) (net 5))
 (segment (start 152.5 72.5) (end 152.5 68) (width 0.25) (layer B.Cu) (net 5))
 (segment (start 171.62 134.62) (end 169.5 132.5) (width 0.25) (layer B.Cu) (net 15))
 (segment (start 171.62 144.5) (end 171.62 134.62) (width 0.25) (layer B.Cu) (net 15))
 (segment (start 169.5 132.5) (end 170 132.5) (width 0.25) (layer F.Cu) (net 15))
 (segment (start 169.5 132.5) (end 169.5 128.886409) (width 0.25) (layer B.Cu) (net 15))
 (segment (start 169.5 128.886409) (end 164.113591 123.5) (width 0.25) (layer B.Cu) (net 15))
 (segment (start 164.113591 123.5) (end 162.5 123.5) (width 0.25) (layer B.Cu) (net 15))
 (segment (start 164 139) (end 160.62 139) (width 0.25) (layer F.Cu) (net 16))
 (segment (start 154.88 129.128996) (end 154.88 128.58) (width 0.25) (layer B.Cu) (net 16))
 (segment (start 160.62 134.868996) (end 154.88 129.128996) (width 0.25) (layer B.Cu) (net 16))
 (segment (start 160.62 139) (end 160.62 134.868996) (width 0.25) (layer B.Cu) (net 16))
 (segment (start 154.58 128.58) (end 154.88 128.58) (width 0.25) (layer F.Cu) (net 16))
 (segment (start 160.62 144.5) (end 160.5 144.5) (width 0.25) (layer B.Cu) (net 8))
 (segment (start 158.5 144.5) (end 153 139) (width 0.25) (layer F.Cu) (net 8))
 (segment (start 160.62 144.5) (end 158.5 144.5) (width 0.25) (layer F.Cu) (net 8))
 (segment (start 153 127.92) (end 154.88 126.04) (width 0.25) (layer B.Cu) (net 8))
 (segment (start 153 139) (end 153 127.92) (width 0.25) (layer B.Cu) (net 8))
 (segment (start 153 40.5) (end 153 41) (width 0.25) (layer F.Cu) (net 12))
 (segment (start 161.245001 60.125001) (end 160.12 59) (width 0.25) (layer B.Cu) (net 12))
 (segment (start 161.245001 71.374999) (end 161.245001 60.125001) (width 0.25) (layer B.Cu) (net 12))
 (segment (start 160.12 72.5) (end 161.245001 71.374999) (width 0.25) (layer B.Cu) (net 12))
 (segment (start 153.5 41) (end 153 41) (width 0.25) (layer B.Cu) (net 12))
 (segment (start 161.69501 42.08818) (end 161.35818 42.42501) (width 0.25) (layer B.Cu) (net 12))
 (segment (start 161.69501 40.424991) (end 161.69501 42.08818) (width 0.25) (layer B.Cu) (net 12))
 (segment (start 163.534989 39.57499) (end 162.545011 39.57499) (width 0.25) (layer B.Cu) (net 12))
 (segment (start 162.545011 39.57499) (end 161.69501 40.424991) (width 0.25) (layer B.Cu) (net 12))
 (segment (start 164.23501 40.275011) (end 163.534989 39.57499) (width 0.25) (layer B.Cu) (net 12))
 (segment (start 154.42501 42.42501) (end 153 41) (width 0.25) (layer B.Cu) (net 12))
 (segment (start 164.23501 46.4414) (end 164.23501 40.275011) (width 0.25) (layer B.Cu) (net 12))
 (segment (start 161.35818 42.42501) (end 154.42501 42.42501) (width 0.25) (layer B.Cu) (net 12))
 (segment (start 160.23501 50.4414) (end 164.23501 46.4414) (width 0.25) (layer B.Cu) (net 12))
 (segment (start 160.23501 58.88499) (end 160.23501 50.4414) (width 0.25) (layer B.Cu) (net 12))
 (segment (start 160.12 59) (end 160.23501 58.88499) (width 0.25) (layer B.Cu) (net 12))
 (segment (start 160.5 40.5) (end 160.5 41) (width 0.25) (layer B.Cu) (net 2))
 (segment (start 160.12 63.5) (end 160.12 63.88) (width 0.25) (layer B.Cu) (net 2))
 (segment (start 160.12 68) (end 160.12 63.88) (width 0.25) (layer B.Cu) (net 2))
 (segment (start 159.07499 39.57499) (end 160.5 41) (width 0.25) (layer F.Cu) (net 2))
 (segment (start 155.045011 39.57499) (end 159.07499 39.57499) (width 0.25) (layer F.Cu) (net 2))
 (segment (start 157.84499 45.224989) (end 154.34499 41.724989) (width 0.25) (layer F.Cu) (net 2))
 (segment (start 157.84499 61.22499) (end 157.84499 45.224989) (width 0.25) (layer F.Cu) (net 2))
 (segment (start 154.34499 40.275011) (end 155.045011 39.57499) (width 0.25) (layer F.Cu) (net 2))
 (segment (start 154.34499 41.724989) (end 154.34499 40.275011) (width 0.25) (layer F.Cu) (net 2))
 (segment (start 160.12 63.5) (end 157.84499 61.22499) (width 0.25) (layer F.Cu) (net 2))
 (segment (start 168 41.095001) (end 168 41) (width 0.25) (layer F.Cu) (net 13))
 (segment (start 172.245001 71.374999) (end 172.245001 45.340002) (width 0.25) (layer B.Cu) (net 13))
 (segment (start 171.12 72.5) (end 172.245001 71.374999) (width 0.25) (layer B.Cu) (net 13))
 (segment (start 172.245001 45.340002) (end 168 41.095001) (width 0.25) (layer B.Cu) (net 13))
 (segment (start 171.12 72.5) (end 171.12 68) (width 0.25) (layer B.Cu) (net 13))
 (segment (start 160 77.5) (end 160.12 77.5) (width 0.25) (layer B.Cu) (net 4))
 (segment (start 169.994999 76.374999) (end 171.12 77.5) (width 0.25) (layer F.Cu) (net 4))
 (segment (start 161.245001 76.374999) (end 169.994999 76.374999) (width 0.25) (layer F.Cu) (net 4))
 (segment (start 160.12 77.5) (end 161.245001 76.374999) (width 0.25) (layer F.Cu) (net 4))
 (segment (start 160.12 77.5) (end 160.5 77.5) (width 0.25) (layer B.Cu) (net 4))
 (segment (start 155.834998 77.5) (end 160.12 77.5) (width 0.25) (layer F.Cu) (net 4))
 (segment (start 151.374999 73.040001) (end 155.834998 77.5) (width 0.25) (layer F.Cu) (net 4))
 (segment (start 151.374999 55.255001) (end 151.374999 73.040001) (width 0.25) (layer F.Cu) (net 4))
 (segment (start 155.63 51) (end 151.374999 55.255001) (width 0.25) (layer F.Cu) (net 4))
 (segment (start 156.5 51) (end 155.63 51) (width 0.25) (layer F.Cu) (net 4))
 (segment (start 171.12 59) (end 164.5 52.38) (width 0.25) (layer B.Cu) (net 3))
 (segment (start 164.5 52.38) (end 164.5 51) (width 0.25) (layer B.Cu) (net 3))
 (segment (start 171.12 59) (end 171.12 63.5) (width 0.25) (layer B.Cu) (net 3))
 (segment (start 154.125001 143.374999) (end 153 144.5) (width 0.25) (layer B.Cu) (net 9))
 (segment (start 164.540001 143.374999) (end 154.125001 143.374999) (width 0.25) (layer B.Cu) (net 9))
 (segment (start 166 144.834998) (end 164.540001 143.374999) (width 0.25) (layer B.Cu) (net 9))
 (segment (start 166 160) (end 166 144.834998) (width 0.25) (layer B.Cu) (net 9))
 (segment (start 156 152.5) (end 164 144.5) (width 0.25) (layer B.Cu) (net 14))
 (segment (start 156 160) (end 156 152.5) (width 0.25) (layer B.Cu) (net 14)))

